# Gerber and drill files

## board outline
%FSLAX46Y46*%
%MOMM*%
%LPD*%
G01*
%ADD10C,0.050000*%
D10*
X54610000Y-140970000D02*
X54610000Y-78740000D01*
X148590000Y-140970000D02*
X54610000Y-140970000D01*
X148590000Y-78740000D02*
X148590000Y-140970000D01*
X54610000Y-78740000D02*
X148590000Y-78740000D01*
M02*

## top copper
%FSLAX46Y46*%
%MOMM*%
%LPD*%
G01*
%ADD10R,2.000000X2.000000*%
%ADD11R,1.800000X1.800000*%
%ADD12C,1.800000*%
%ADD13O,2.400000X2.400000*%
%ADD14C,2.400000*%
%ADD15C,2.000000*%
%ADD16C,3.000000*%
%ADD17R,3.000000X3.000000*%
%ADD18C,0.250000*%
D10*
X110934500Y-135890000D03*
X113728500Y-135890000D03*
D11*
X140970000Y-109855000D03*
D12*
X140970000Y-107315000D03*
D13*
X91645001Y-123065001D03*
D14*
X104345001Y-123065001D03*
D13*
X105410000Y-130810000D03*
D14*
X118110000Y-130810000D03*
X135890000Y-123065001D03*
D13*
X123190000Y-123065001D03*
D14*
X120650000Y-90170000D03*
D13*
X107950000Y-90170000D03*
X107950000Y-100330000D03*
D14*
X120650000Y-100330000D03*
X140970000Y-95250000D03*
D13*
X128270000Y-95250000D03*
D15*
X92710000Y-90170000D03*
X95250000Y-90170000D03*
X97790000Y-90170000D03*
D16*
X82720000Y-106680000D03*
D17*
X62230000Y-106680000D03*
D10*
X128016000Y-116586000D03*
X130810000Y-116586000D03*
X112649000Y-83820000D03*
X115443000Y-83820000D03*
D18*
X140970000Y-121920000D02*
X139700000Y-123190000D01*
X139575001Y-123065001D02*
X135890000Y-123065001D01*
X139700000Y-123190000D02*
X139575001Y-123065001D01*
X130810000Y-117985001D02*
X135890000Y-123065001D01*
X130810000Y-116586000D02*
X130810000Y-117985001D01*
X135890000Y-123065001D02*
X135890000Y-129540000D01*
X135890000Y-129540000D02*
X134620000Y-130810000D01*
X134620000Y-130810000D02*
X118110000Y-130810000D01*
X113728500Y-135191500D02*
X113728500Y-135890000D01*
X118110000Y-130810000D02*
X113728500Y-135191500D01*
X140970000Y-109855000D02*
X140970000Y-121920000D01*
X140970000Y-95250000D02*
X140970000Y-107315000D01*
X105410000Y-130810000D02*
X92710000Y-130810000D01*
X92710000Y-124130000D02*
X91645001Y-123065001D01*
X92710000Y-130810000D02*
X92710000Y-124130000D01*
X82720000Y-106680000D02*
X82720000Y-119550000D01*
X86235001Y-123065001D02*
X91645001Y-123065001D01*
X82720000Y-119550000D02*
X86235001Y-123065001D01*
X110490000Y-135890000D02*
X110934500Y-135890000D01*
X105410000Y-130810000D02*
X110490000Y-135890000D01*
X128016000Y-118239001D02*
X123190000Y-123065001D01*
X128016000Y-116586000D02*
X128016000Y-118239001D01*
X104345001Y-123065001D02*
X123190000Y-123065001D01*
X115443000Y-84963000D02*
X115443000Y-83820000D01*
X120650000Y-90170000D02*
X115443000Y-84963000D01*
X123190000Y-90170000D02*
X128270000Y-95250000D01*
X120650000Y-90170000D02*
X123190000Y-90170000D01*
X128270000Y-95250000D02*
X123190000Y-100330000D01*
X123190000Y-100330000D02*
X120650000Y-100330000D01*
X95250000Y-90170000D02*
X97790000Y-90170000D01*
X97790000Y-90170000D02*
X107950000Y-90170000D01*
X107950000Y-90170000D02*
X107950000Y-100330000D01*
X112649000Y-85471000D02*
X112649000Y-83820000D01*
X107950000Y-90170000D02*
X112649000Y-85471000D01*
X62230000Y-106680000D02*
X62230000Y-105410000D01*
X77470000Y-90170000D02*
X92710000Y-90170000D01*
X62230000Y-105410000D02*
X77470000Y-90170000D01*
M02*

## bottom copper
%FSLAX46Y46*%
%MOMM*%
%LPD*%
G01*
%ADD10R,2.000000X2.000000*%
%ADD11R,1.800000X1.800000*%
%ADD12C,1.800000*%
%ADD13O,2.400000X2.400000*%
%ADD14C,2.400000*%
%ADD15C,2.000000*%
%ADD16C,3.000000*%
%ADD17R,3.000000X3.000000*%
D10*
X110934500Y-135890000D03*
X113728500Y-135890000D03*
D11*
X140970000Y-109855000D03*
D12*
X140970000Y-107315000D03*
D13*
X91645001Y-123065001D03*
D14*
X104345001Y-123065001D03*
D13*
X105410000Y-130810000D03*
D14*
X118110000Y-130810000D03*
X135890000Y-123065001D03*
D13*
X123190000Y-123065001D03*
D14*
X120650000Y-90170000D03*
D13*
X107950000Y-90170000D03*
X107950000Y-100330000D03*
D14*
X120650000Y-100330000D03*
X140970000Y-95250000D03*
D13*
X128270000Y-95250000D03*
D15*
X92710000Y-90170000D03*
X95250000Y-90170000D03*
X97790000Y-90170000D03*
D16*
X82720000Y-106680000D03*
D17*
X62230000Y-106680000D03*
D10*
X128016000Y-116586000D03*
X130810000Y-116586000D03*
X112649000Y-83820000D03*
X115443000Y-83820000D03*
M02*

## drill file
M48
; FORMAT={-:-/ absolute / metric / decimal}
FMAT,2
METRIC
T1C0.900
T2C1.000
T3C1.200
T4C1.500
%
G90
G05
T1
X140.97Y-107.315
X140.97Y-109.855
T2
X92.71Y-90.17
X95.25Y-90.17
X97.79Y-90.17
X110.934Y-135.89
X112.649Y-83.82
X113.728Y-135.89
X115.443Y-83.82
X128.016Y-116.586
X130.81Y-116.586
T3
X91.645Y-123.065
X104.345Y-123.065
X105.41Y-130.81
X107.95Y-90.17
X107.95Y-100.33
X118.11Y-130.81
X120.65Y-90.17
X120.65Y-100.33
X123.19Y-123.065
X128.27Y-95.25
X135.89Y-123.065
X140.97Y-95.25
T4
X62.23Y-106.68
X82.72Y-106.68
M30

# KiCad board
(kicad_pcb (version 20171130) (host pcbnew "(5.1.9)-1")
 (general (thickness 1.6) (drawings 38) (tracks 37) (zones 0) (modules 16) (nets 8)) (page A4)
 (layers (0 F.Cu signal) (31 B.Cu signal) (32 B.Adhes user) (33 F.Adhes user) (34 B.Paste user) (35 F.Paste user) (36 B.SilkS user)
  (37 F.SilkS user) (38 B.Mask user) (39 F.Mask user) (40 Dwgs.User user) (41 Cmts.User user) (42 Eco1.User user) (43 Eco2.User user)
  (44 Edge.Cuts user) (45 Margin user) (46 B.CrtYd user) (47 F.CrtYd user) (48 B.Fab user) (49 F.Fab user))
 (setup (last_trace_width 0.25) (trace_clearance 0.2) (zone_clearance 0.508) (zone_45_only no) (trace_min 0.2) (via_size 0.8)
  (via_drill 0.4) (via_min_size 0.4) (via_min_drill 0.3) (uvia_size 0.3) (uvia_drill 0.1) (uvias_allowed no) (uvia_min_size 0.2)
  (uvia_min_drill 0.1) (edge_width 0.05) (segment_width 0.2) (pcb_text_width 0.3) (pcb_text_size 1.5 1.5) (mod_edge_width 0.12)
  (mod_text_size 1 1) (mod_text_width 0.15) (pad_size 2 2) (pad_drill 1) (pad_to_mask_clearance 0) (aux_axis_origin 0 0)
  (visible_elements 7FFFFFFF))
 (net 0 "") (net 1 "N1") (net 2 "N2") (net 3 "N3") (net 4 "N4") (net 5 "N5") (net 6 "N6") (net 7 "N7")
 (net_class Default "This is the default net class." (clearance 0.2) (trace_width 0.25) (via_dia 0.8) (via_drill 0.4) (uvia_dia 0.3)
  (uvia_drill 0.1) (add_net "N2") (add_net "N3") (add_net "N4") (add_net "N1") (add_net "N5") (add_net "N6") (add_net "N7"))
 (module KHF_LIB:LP (layer F.Cu) (at 110.9345 135.89)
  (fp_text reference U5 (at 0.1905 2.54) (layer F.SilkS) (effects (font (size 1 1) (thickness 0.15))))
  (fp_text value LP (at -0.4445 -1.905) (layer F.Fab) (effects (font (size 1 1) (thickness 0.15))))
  (pad 1 thru_hole rect (at 0 0) (size 2 2) (drill 1) (layers *.Cu *.Mask) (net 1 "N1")))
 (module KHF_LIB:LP (layer F.Cu) (at 113.7285 135.89)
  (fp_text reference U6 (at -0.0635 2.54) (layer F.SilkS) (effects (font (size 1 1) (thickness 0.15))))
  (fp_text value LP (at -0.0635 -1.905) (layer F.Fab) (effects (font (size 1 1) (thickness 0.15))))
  (pad 1 thru_hole rect (at 0 0) (size 2 2) (drill 1) (layers *.Cu *.Mask) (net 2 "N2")))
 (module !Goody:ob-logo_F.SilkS (layer F.Cu) (at 111.76 111.76)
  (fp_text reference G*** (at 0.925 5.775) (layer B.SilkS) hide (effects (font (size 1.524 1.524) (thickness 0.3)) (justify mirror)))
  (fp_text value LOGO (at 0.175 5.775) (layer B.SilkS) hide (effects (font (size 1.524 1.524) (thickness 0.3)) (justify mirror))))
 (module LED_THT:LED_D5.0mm (layer F.Cu) (at 140.97 109.855 90)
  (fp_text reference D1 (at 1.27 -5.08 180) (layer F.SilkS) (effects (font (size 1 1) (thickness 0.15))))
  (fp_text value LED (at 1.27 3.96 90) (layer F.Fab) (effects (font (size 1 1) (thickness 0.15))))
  (pad 1 thru_hole rect (at 0 0 90) (size 1.8 1.8) (drill 0.9) (layers *.Cu *.Mask) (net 2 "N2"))
  (pad 2 thru_hole circle (at 2.54 0 90) (size 1.8 1.8) (drill 0.9) (layers *.Cu *.Mask) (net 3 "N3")))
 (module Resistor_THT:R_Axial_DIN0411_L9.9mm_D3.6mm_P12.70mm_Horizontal (layer F.Cu) (at 104.345001 123.065001 180)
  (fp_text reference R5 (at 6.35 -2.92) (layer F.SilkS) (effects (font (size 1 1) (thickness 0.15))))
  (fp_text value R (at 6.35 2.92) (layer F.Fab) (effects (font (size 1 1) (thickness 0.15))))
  (pad 2 thru_hole oval (at 12.7 0 180) (size 2.4 2.4) (drill 1.2) (layers *.Cu *.Mask) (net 1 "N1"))
  (pad 1 thru_hole circle (at 0 0 180) (size 2.4 2.4) (drill 1.2) (layers *.Cu *.Mask) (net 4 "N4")))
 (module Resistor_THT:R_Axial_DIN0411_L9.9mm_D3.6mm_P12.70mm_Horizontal (layer F.Cu) (at 118.11 130.81 180)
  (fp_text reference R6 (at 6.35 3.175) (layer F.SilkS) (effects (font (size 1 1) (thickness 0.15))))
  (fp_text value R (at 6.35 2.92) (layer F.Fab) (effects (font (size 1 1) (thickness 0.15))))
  (pad 2 thru_hole oval (at 12.7 0 180) (size 2.4 2.4) (drill 1.2) (layers *.Cu *.Mask) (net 1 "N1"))
  (pad 1 thru_hole circle (at 0 0 180) (size 2.4 2.4) (drill 1.2) (layers *.Cu *.Mask) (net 2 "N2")))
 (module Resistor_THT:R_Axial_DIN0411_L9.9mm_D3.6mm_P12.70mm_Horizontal (layer F.Cu) (at 135.89 123.065001 180)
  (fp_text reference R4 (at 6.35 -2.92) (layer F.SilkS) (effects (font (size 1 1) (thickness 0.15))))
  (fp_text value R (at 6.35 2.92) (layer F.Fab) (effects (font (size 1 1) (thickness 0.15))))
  (pad 1 thru_hole circle (at 0 0 180) (size 2.4 2.4) (drill 1.2) (layers *.Cu *.Mask) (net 2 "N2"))
  (pad 2 thru_hole oval (at 12.7 0 180) (size 2.4 2.4) (drill 1.2) (layers *.Cu *.Mask) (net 4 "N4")))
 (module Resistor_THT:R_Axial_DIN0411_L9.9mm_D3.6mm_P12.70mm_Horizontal (layer F.Cu) (at 120.65 90.17 180)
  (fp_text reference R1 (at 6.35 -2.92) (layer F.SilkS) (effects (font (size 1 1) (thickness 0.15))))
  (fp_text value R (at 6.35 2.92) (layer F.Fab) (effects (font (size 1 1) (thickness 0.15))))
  (pad 1 thru_hole circle (at 0 0 180) (size 2.4 2.4) (drill 1.2) (layers *.Cu *.Mask) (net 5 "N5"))
  (pad 2 thru_hole oval (at 12.7 0 180) (size 2.4 2.4) (drill 1.2) (layers *.Cu *.Mask) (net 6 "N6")))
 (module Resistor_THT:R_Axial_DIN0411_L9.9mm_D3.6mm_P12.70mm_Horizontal (layer F.Cu) (at 120.65 100.33 180)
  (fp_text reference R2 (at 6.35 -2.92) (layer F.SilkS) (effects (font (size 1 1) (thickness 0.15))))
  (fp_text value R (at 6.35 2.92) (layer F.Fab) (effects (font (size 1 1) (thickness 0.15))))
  (pad 2 thru_hole oval (at 12.7 0 180) (size 2.4 2.4) (drill 1.2) (layers *.Cu *.Mask) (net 6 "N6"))
  (pad 1 thru_hole circle (at 0 0 180) (size 2.4 2.4) (drill 1.2) (layers *.Cu *.Mask) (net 5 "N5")))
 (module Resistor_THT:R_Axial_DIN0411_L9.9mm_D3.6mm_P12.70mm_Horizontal (layer F.Cu) (at 140.97 95.25 180)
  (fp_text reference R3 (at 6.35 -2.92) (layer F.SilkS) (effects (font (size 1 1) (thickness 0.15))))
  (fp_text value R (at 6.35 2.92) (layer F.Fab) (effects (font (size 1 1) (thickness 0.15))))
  (pad 1 thru_hole circle (at 0 0 180) (size 2.4 2.4) (drill 1.2) (layers *.Cu *.Mask) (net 3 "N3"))
  (pad 2 thru_hole oval (at 12.7 0 180) (size 2.4 2.4) (drill 1.2) (layers *.Cu *.Mask) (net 5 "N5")))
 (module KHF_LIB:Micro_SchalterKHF (layer F.Cu) (at 92.71 90.17)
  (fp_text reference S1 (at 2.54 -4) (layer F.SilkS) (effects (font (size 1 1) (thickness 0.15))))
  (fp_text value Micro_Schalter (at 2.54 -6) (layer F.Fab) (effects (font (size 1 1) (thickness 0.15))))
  (pad 1 thru_hole circle (at 0 0) (size 2 2) (drill 1) (layers *.Cu *.Mask) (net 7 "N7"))
  (pad 2 thru_hole circle (at 2.54 0) (size 2 2) (drill 1) (layers *.Cu *.Mask) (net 6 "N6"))
  (pad 3 thru_hole circle (at 5.08 0) (size 2 2) (drill 1) (layers *.Cu *.Mask) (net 6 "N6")))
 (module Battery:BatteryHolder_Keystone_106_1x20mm (layer F.Cu) (at 62.23 106.68)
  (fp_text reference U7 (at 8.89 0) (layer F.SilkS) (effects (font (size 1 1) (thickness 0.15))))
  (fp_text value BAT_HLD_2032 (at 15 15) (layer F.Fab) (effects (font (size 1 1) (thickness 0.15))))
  (pad 2 thru_hole circle (at 20.49 0) (size 3 3) (drill 1.5) (layers *.Cu *.Mask) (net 1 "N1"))
  (pad 1 thru_hole rect (at 0 0) (size 3 3) (drill 1.5) (layers *.Cu *.Mask) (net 7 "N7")))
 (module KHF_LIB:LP (layer F.Cu) (at 128.016 116.586)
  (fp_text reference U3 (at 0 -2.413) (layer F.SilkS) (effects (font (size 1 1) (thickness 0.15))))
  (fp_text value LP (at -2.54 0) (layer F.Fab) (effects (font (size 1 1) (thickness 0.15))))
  (pad 1 thru_hole rect (at 0 0) (size 2 2) (drill 1) (layers *.Cu *.Mask) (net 4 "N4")))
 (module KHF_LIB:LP (layer F.Cu) (at 130.81 116.586)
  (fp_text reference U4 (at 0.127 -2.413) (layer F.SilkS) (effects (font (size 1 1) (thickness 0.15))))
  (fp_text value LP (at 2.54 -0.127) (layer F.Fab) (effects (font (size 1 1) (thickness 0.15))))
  (pad 1 thru_hole rect (at 0 0) (size 2 2) (drill 1) (layers *.Cu *.Mask) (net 2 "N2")))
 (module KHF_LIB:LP (layer F.Cu) (at 112.649 83.82)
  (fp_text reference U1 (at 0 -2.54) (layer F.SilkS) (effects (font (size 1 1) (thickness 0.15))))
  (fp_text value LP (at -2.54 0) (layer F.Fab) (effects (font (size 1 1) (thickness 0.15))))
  (pad 1 thru_hole rect (at 0 0) (size 2 2) (drill 1) (layers *.Cu *.Mask) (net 6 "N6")))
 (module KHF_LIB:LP (layer F.Cu) (at 115.443 83.82)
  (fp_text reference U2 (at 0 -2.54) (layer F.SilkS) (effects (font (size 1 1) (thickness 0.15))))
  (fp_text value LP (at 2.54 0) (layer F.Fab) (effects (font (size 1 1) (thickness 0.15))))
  (pad 1 thru_hole rect (at 0 0) (size 2 2) (drill 1) (layers *.Cu *.Mask) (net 5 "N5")))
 (gr_line (start 54.61 140.97) (end 54.61 78.74) (layer Edge.Cuts) (width 0.05))
 (gr_line (start 148.59 140.97) (end 54.61 140.97) (layer Edge.Cuts) (width 0.05))
 (gr_line (start 148.59 78.74) (end 148.59 140.97) (layer Edge.Cuts) (width 0.05))
 (gr_line (start 54.61 78.74) (end 148.59 78.74) (layer Edge.Cuts) (width 0.05))
 (segment (start 140.97 121.92) (end 139.7 123.19) (width 0.25) (layer F.Cu) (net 2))
 (segment (start 139.575001 123.065001) (end 135.89 123.065001) (width 0.25) (layer F.Cu) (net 2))
 (segment (start 139.7 123.19) (end 139.575001 123.065001) (width 0.25) (layer F.Cu) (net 2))
 (segment (start 130.81 117.985001) (end 135.89 123.065001) (width 0.25) (layer F.Cu) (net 2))
 (segment (start 130.81 116.586) (end 130.81 117.985001) (width 0.25) (layer F.Cu) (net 2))
 (segment (start 135.89 123.065001) (end 135.89 129.54) (width 0.25) (layer F.Cu) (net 2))
 (segment (start 135.89 129.54) (end 134.62 130.81) (width 0.25) (layer F.Cu) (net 2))
 (segment (start 134.62 130.81) (end 118.11 130.81) (width 0.25) (layer F.Cu) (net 2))
 (segment (start 113.7285 135.1915) (end 113.7285 135.89) (width 0.25) (layer F.Cu) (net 2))
 (segment (start 118.11 130.81) (end 113.7285 135.1915) (width 0.25) (layer F.Cu) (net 2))
 (segment (start 140.97 109.855) (end 140.97 121.92) (width 0.25) (layer F.Cu) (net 2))
 (segment (start 140.97 95.25) (end 140.97 107.315) (width 0.25) (layer F.Cu) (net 3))
 (segment (start 105.41 130.81) (end 92.71 130.81) (width 0.25) (layer F.Cu) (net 1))
 (segment (start 92.71 124.13) (end 91.645001 123.065001) (width 0.25) (layer F.Cu) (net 1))
 (segment (start 92.71 130.81) (end 92.71 124.13) (width 0.25) (layer F.Cu) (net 1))
 (segment (start 82.72 106.68) (end 82.72 119.55) (width 0.25) (layer F.Cu) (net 1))
 (segment (start 86.235001 123.065001) (end 91.645001 123.065001) (width 0.25) (layer F.Cu) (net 1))
 (segment (start 82.72 119.55) (end 86.235001 123.065001) (width 0.25) (layer F.Cu) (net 1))
 (segment (start 110.49 135.89) (end 110.9345 135.89) (width 0.25) (layer F.Cu) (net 1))
 (segment (start 105.41 130.81) (end 110.49 135.89) (width 0.25) (layer F.Cu) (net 1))
 (segment (start 128.016 118.239001) (end 123.19 123.065001) (width 0.25) (layer F.Cu) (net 4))
 (segment (start 128.016 116.586) (end 128.016 118.239001) (width 0.25) (layer F.Cu) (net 4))
 (segment (start 104.345001 123.065001) (end 123.19 123.065001) (width 0.25) (layer F.Cu) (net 4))
 (segment (start 115.443 84.963) (end 115.443 83.82) (width 0.25) (layer F.Cu) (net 5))
 (segment (start 120.65 90.17) (end 115.443 84.963) (width 0.25) (layer F.Cu) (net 5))
 (segment (start 123.19 90.17) (end 128.27 95.25) (width 0.25) (layer F.Cu) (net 5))
 (segment (start 120.65 90.17) (end 123.19 90.17) (width 0.25) (layer F.Cu) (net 5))
 (segment (start 128.27 95.25) (end 123.19 100.33) (width 0.25) (layer F.Cu) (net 5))
 (segment (start 123.19 100.33) (end 120.65 100.33) (width 0.25) (layer F.Cu) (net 5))
 (segment (start 95.25 90.17) (end 97.79 90.17) (width 0.25) (layer F.Cu) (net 6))
 (segment (start 97.79 90.17) (end 107.95 90.17) (width 0.25) (layer F.Cu) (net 6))
 (segment (start 107.95 90.17) (end 107.95 100.33) (width 0.25) (layer F.Cu) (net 6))
 (segment (start 112.649 85.471) (end 112.649 83.82) (width 0.25) (layer F.Cu) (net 6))
 (segment (start 107.95 90.17) (end 112.649 85.471) (width 0.25) (layer F.Cu) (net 6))
 (segment (start 62.23 106.68) (end 62.23 105.41) (width 0.25) (layer F.Cu) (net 7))
 (segment (start 77.47 90.17) (end 92.71 90.17) (width 0.25) (layer F.Cu) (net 7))
 (segment (start 62.23 105.41) (end 77.47 90.17) (width 0.25) (layer F.Cu) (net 7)))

